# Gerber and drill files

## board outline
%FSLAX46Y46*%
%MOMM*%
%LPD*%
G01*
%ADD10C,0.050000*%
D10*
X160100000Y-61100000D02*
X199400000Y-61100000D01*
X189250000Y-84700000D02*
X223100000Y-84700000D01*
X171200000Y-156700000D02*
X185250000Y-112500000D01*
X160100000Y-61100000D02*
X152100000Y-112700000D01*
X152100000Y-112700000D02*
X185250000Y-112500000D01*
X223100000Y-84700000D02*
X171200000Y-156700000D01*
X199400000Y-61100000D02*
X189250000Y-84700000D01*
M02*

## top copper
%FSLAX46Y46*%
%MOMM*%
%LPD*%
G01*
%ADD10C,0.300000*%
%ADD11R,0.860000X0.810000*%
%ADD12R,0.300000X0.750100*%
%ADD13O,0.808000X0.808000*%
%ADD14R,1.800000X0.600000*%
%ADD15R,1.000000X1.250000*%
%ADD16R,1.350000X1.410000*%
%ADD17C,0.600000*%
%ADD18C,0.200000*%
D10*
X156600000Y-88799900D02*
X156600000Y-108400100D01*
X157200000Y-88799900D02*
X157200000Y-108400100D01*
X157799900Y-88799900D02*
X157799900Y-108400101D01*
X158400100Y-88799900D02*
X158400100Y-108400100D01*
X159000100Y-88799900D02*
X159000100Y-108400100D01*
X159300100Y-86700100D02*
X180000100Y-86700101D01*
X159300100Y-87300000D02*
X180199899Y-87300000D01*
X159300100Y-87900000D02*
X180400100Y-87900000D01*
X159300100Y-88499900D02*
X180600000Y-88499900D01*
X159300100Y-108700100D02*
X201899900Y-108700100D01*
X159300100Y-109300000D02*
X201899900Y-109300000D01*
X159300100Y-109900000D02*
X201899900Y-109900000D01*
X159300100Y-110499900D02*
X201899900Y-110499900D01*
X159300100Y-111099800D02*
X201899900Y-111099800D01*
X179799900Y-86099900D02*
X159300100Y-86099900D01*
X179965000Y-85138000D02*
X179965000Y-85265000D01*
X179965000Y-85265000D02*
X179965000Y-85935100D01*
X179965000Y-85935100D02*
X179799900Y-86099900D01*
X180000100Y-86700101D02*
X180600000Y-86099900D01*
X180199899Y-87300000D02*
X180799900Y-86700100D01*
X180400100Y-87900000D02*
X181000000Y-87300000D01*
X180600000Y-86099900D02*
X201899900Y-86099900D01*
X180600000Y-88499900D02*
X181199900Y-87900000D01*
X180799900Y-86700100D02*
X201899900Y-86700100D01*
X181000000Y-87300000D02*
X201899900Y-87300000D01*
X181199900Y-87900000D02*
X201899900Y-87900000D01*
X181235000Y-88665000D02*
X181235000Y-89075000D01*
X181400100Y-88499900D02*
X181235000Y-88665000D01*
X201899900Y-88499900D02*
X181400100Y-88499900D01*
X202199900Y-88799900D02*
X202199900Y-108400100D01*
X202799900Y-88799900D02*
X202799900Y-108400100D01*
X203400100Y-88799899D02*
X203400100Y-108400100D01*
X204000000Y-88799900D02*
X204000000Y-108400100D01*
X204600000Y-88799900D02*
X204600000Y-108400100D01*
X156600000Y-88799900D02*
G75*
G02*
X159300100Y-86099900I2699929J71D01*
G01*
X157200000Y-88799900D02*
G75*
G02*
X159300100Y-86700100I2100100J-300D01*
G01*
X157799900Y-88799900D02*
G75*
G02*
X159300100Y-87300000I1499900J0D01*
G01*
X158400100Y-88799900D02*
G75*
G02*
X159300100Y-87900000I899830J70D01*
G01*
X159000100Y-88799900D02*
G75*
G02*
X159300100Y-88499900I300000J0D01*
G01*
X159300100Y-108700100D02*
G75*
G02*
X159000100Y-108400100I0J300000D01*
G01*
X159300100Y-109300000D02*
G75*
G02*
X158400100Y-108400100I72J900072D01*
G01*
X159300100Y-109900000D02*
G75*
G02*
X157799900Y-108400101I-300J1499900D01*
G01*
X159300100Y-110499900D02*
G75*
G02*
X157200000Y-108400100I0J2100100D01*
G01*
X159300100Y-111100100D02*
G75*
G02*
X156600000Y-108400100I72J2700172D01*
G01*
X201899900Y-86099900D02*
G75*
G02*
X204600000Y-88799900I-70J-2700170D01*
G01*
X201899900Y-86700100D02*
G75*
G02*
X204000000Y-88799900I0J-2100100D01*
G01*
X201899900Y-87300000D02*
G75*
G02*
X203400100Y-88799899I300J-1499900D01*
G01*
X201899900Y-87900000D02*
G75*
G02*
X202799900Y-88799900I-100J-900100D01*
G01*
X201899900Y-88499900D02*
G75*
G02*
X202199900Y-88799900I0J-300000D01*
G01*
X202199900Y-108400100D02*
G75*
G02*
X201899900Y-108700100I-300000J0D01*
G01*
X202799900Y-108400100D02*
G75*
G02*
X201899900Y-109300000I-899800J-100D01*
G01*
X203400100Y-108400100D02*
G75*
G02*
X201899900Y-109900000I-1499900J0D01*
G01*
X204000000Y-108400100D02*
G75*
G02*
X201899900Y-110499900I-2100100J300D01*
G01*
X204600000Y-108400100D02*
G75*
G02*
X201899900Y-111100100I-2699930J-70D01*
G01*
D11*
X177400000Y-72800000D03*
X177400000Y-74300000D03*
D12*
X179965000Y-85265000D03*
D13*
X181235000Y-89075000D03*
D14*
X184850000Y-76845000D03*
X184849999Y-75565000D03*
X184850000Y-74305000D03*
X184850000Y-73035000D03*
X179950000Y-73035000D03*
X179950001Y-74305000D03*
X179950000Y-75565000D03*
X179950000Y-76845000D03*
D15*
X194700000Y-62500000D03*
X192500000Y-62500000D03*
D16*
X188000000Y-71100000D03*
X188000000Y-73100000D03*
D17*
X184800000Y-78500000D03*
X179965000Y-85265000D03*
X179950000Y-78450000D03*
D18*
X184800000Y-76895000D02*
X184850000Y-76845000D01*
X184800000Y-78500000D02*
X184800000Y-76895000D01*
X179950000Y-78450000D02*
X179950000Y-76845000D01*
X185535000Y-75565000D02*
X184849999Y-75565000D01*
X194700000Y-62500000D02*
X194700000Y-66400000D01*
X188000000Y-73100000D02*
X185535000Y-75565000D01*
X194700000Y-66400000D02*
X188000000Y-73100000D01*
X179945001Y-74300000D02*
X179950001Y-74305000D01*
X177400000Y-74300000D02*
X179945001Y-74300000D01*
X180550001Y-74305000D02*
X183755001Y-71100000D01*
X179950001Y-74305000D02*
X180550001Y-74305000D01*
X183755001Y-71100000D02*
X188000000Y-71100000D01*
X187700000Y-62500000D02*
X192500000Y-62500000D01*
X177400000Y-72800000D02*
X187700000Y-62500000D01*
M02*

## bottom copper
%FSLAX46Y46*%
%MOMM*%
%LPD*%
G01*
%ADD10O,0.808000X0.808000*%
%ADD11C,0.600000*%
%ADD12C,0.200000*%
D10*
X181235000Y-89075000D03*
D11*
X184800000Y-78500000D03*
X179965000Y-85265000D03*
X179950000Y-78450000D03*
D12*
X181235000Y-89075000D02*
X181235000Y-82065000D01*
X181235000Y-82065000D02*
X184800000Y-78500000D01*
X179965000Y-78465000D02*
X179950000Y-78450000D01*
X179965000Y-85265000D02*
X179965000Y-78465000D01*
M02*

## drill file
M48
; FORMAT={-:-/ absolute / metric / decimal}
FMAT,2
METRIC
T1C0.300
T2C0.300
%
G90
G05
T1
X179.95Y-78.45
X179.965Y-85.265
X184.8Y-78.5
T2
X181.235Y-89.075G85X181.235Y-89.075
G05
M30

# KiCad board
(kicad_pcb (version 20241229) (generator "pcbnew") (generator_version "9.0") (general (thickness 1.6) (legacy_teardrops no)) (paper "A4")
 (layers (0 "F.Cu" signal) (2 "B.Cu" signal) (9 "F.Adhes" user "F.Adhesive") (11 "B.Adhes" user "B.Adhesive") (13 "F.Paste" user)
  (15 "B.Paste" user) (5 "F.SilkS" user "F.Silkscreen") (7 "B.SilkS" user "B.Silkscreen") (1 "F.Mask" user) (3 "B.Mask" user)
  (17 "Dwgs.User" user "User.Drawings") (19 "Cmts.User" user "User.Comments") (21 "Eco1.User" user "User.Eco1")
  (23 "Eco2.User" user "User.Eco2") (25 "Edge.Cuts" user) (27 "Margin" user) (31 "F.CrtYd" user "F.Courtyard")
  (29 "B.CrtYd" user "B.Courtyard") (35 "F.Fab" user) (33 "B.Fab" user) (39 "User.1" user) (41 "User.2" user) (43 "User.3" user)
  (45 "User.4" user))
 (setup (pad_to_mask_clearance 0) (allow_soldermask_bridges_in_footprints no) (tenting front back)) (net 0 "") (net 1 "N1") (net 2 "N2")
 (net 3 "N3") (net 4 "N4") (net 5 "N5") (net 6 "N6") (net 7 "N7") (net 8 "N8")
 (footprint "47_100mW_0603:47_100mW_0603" (layer "F.Cu") (at 177.4 73.55 -90)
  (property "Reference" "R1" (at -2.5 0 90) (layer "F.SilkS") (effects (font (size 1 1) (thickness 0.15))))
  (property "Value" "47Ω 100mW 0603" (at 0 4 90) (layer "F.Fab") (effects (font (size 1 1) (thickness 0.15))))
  (pad "1" smd rect (at -0.75 0 270) (size 0.81 0.86) (layers "F.Cu" "F.Mask" "F.Paste") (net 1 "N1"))
  (pad "2" smd rect (at 0.75 0 270) (size 0.81 0.86) (layers "F.Cu" "F.Mask" "F.Paste") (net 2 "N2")))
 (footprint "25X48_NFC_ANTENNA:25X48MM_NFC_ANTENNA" (layer "F.Cu") (at 180.6 98.6)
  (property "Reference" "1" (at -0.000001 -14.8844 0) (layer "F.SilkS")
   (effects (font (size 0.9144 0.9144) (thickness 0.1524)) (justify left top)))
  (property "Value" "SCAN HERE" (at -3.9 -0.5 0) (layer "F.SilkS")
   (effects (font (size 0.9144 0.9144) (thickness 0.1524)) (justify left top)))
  (fp_line (start -24 -9.8001) (end -24 9.8001) (stroke (width 0.3) (type default)) (layer "F.Cu"))
  (fp_line (start -23.4 -9.8001) (end -23.4 9.8001) (stroke (width 0.3) (type default)) (layer "F.Cu"))
  (fp_line (start -22.8001 -9.8001) (end -22.8001 9.800101) (stroke (width 0.3) (type default)) (layer "F.Cu"))
  (fp_line (start -22.1999 -9.8001) (end -22.1999 9.8001) (stroke (width 0.3) (type default)) (layer "F.Cu"))
  (fp_line (start -21.5999 -9.8001) (end -21.5999 9.8001) (stroke (width 0.3) (type default)) (layer "F.Cu"))
  (fp_line (start -21.2999 -11.8999) (end -0.5999 -11.899899) (stroke (width 0.3) (type default)) (layer "F.Cu"))
  (fp_line (start -21.2999 -11.3) (end -0.400101 -11.3) (stroke (width 0.3) (type default)) (layer "F.Cu"))
  (fp_line (start -21.2999 -10.7) (end -0.1999 -10.7) (stroke (width 0.3) (type default)) (layer "F.Cu"))
  (fp_line (start -21.2999 -10.1001) (end 0 -10.1001) (stroke (width 0.3) (type default)) (layer "F.Cu"))
  (fp_line (start -21.2999 10.1001) (end 21.2999 10.1001) (stroke (width 0.3) (type default)) (layer "F.Cu"))
  (fp_line (start -21.2999 10.7) (end 21.2999 10.7) (stroke (width 0.3) (type default)) (layer "F.Cu"))
  (fp_line (start -21.2999 11.3) (end 21.2999 11.3) (stroke (width 0.3) (type default)) (layer "F.Cu"))
  (fp_line (start -21.2999 11.8999) (end 21.2999 11.8999) (stroke (width 0.3) (type default)) (layer "F.Cu"))
  (fp_line (start -21.2999 12.4998) (end 21.2999 12.4998) (stroke (width 0.3) (type default)) (layer "F.Cu"))
  (fp_line (start -0.8001 -12.5001) (end -21.2999 -12.5001) (stroke (width 0.3) (type default)) (layer "F.Cu"))
  (fp_line (start -0.635 -13.462) (end -0.635 -13.335) (stroke (width 0.3) (type default)) (layer "F.Cu"))
  (fp_line (start -0.635 -13.335) (end -0.635 -12.6649) (stroke (width 0.3) (type default)) (layer "F.Cu"))
  (fp_line (start -0.635 -12.6649) (end -0.8001 -12.5001) (stroke (width 0.3) (type default)) (layer "F.Cu"))
  (fp_line (start -0.5999 -11.899899) (end 0 -12.5001) (stroke (width 0.3) (type default)) (layer "F.Cu"))
  (fp_line (start -0.400101 -11.3) (end 0.1999 -11.8999) (stroke (width 0.3) (type default)) (layer "F.Cu"))
  (fp_line (start -0.1999 -10.7) (end 0.4 -11.3) (stroke (width 0.3) (type default)) (layer "F.Cu"))
  (fp_line (start 0 -12.5001) (end 21.2999 -12.5001) (stroke (width 0.3) (type default)) (layer "F.Cu"))
  (fp_line (start 0 -10.1001) (end 0.5999 -10.7) (stroke (width 0.3) (type default)) (layer "F.Cu"))
  (fp_line (start 0.1999 -11.8999) (end 21.2999 -11.8999) (stroke (width 0.3) (type default)) (layer "F.Cu"))
  (fp_line (start 0.4 -11.3) (end 21.2999 -11.3) (stroke (width 0.3) (type default)) (layer "F.Cu"))
  (fp_line (start 0.5999 -10.7) (end 21.2999 -10.7) (stroke (width 0.3) (type default)) (layer "F.Cu"))
  (fp_line (start 0.635 -9.935) (end 0.635 -9.525) (stroke (width 0.3) (type default)) (layer "F.Cu"))
  (fp_line (start 0.8001 -10.1001) (end 0.635 -9.935) (stroke (width 0.3) (type default)) (layer "F.Cu"))
  (fp_line (start 21.2999 -10.1001) (end 0.8001 -10.1001) (stroke (width 0.3) (type default)) (layer "F.Cu"))
  (fp_line (start 21.5999 -9.8001) (end 21.5999 9.8001) (stroke (width 0.3) (type default)) (layer "F.Cu"))
  (fp_line (start 22.1999 -9.8001) (end 22.1999 9.8001) (stroke (width 0.3) (type default)) (layer "F.Cu"))
  (fp_line (start 22.8001 -9.800101) (end 22.8001 9.8001) (stroke (width 0.3) (type default)) (layer "F.Cu"))
  (fp_line (start 23.4 -9.8001) (end 23.4 9.8001) (stroke (width 0.3) (type default)) (layer "F.Cu"))
  (fp_line (start 24 -9.8001) (end 24 9.8001) (stroke (width 0.3) (type default)) (layer "F.Cu"))
  (fp_arc (start -24 -9.8001) (mid -23.209159 -11.709359) (end -21.2999 -12.5001) (stroke (width 0.3) (type default)) (layer "F.Cu"))
  (fp_arc (start -23.4 -9.8001) (mid -22.784789 -11.284901) (end -21.2999 -11.8999) (stroke (width 0.3) (type default)) (layer "F.Cu"))
  (fp_arc (start -22.8001 -9.8001) (mid -22.360683 -10.860796) (end -21.2999 -11.3) (stroke (width 0.3) (type default)) (layer "F.Cu"))
  (fp_arc (start -22.1999 -9.8001) (mid -21.936296 -10.436496) (end -21.2999 -10.7) (stroke (width 0.3) (type default)) (layer "F.Cu"))
  (fp_arc (start -21.5999 -9.8001) (mid -21.512032 -10.012232) (end -21.2999 -10.1001) (stroke (width 0.3) (type default)) (layer "F.Cu"))
  (fp_arc (start -21.2999 10.1001) (mid -21.512032 10.012232) (end -21.5999 9.8001) (stroke (width 0.3) (type default)) (layer "F.Cu"))
  (fp_arc (start -21.2999 10.7) (mid -21.936225 10.436425) (end -22.1999 9.8001) (stroke (width 0.3) (type default)) (layer "F.Cu"))
  (fp_arc (start -21.2999 11.3) (mid -22.360683 10.860796) (end -22.8001 9.800101) (stroke (width 0.3) (type default)) (layer "F.Cu"))
  (fp_arc (start -21.2999 11.8999) (mid -22.784789 11.284901) (end -23.4 9.8001) (stroke (width 0.3) (type default)) (layer "F.Cu"))
  (fp_arc (start -21.2999 12.5001) (mid -23.209088 11.709288) (end -24 9.8001) (stroke (width 0.3) (type default)) (layer "F.Cu"))
  (fp_arc (start 21.2999 -12.5001) (mid 23.209088 -11.709288) (end 24 -9.8001) (stroke (width 0.3) (type default)) (layer "F.Cu"))
  (fp_arc (start 21.2999 -11.8999) (mid 22.784789 -11.284901) (end 23.4 -9.8001) (stroke (width 0.3) (type default)) (layer "F.Cu"))
  (fp_arc (start 21.2999 -11.3) (mid 22.360683 -10.860796) (end 22.8001 -9.800101) (stroke (width 0.3) (type default)) (layer "F.Cu"))
  (fp_arc (start 21.2999 -10.7) (mid 21.936225 -10.436425) (end 22.1999 -9.8001) (stroke (width 0.3) (type default)) (layer "F.Cu"))
  (fp_arc (start 21.2999 -10.1001) (mid 21.512032 -10.012232) (end 21.5999 -9.8001) (stroke (width 0.3) (type default)) (layer "F.Cu"))
  (fp_arc (start 21.5999 9.8001) (mid 21.512032 10.012232) (end 21.2999 10.1001) (stroke (width 0.3) (type default)) (layer "F.Cu"))
  (fp_arc (start 22.1999 9.8001) (mid 21.936296 10.436496) (end 21.2999 10.7) (stroke (width 0.3) (type default)) (layer "F.Cu"))
  (fp_arc (start 22.8001 9.8001) (mid 22.360683 10.860796) (end 21.2999 11.3) (stroke (width 0.3) (type default)) (layer "F.Cu"))
  (fp_arc (start 23.4 9.8001) (mid 22.784789 11.284901) (end 21.2999 11.8999) (stroke (width 0.3) (type default)) (layer "F.Cu"))
  (fp_arc (start 24 9.8001) (mid 23.209159 11.709359) (end 21.2999 12.5001) (stroke (width 0.3) (type default)) (layer "F.Cu"))
  (pad "P$1" smd rect (at -0.635 -13.335 90) (size 0.7501 0.3) (layers "F.Cu" "F.Mask" "F.Paste") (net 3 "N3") (solder_mask_margin 0.0508)
   (solder_paste_margin 0) (thermal_bridge_angle 0))
  (pad "P$2" thru_hole oval (at 0.635 -9.525) (size 0.808 0.808) (drill oval 0.3005 0.3002) (layers "*.Cu" "*.Mask")
   (remove_unused_layers no) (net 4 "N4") (solder_mask_margin 0.0508) (solder_paste_margin 0) (thermal_bridge_angle 0)))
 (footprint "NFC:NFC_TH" (layer "F.Cu") (at 182.4 74.935 90)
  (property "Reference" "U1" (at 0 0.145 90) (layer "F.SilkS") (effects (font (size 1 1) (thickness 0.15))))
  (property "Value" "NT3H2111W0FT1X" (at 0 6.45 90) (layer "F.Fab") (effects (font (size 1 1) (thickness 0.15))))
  (pad "1" smd rect (at -1.91 2.45 90) (size 0.6 1.8) (layers "F.Cu" "F.Mask" "F.Paste") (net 4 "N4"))
  (pad "2" smd rect (at -0.63 2.449999 90) (size 0.6 1.8) (layers "F.Cu" "F.Mask" "F.Paste") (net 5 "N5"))
  (pad "3" smd rect (at 0.63 2.45 90) (size 0.6 1.8) (layers "F.Cu" "F.Mask" "F.Paste") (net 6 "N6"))
  (pad "4" smd rect (at 1.9 2.45 90) (size 0.6 1.8) (layers "F.Cu" "F.Mask" "F.Paste") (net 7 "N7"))
  (pad "5" smd rect (at 1.9 -2.45 270) (size 0.6 1.8) (layers "F.Cu" "F.Mask" "F.Paste") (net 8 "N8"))
  (pad "6" smd rect (at 0.63 -2.449999 270) (size 0.6 1.8) (layers "F.Cu" "F.Mask" "F.Paste") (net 2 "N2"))
  (pad "7" smd rect (at -0.63 -2.45 270) (size 0.6 1.8) (layers "F.Cu" "F.Mask" "F.Paste") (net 2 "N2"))
  (pad "8" smd rect (at -1.91 -2.45 270) (size 0.6 1.8) (layers "F.Cu" "F.Mask" "F.Paste") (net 3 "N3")))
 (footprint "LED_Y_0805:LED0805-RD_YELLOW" (layer "F.Cu") (at 193.6 62.5 180)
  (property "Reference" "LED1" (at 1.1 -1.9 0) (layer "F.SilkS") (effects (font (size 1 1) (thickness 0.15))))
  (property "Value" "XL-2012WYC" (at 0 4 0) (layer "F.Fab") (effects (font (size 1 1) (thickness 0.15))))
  (pad "1" smd rect (at -1.1 0) (size 1 1.25) (layers "F.Cu" "F.Mask" "F.Paste") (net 5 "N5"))
  (pad "2" smd rect (at 1.1 0) (size 1 1.25) (layers "F.Cu" "F.Mask" "F.Paste") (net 1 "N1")))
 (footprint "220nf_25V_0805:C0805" (layer "F.Cu") (at 188 72.1 -90)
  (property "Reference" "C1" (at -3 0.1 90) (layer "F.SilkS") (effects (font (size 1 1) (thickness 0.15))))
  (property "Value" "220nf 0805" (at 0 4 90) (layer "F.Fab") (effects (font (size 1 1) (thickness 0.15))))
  (pad "1" smd rect (at -1 0 270) (size 1.41 1.35) (layers "F.Cu" "F.Mask" "F.Paste") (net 2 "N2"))
  (pad "2" smd rect (at 1 0 270) (size 1.41 1.35) (layers "F.Cu" "F.Mask" "F.Paste") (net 5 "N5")))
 (gr_line (start 160.1 61.1) (end 199.4 61.1) (stroke (width 0.05) (type default)) (layer "Edge.Cuts"))
 (gr_line (start 189.25 84.7) (end 223.1 84.7) (stroke (width 0.05) (type default)) (layer "Edge.Cuts"))
 (gr_line (start 171.2 156.7) (end 185.25 112.5) (stroke (width 0.05) (type default)) (layer "Edge.Cuts"))
 (gr_line (start 160.1 61.1) (end 152.1 112.7) (stroke (width 0.05) (type default)) (layer "Edge.Cuts"))
 (gr_line (start 152.1 112.7) (end 185.25 112.5) (stroke (width 0.05) (type default)) (layer "Edge.Cuts"))
 (gr_line (start 223.1 84.7) (end 171.2 156.7) (stroke (width 0.05) (type default)) (layer "Edge.Cuts"))
 (gr_line (start 199.4 61.1) (end 189.25 84.7) (stroke (width 0.05) (type default)) (layer "Edge.Cuts"))
 (segment (start 184.8 76.895) (end 184.85 76.845) (width 0.2) (layer "F.Cu") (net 4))
 (segment (start 184.8 78.5) (end 184.8 76.895) (width 0.2) (layer "F.Cu") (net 4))
 (via (at 184.8 78.5) (size 0.6) (drill 0.3) (layers "F.Cu" "B.Cu") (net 4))
 (segment (start 181.235 89.075) (end 181.235 82.065) (width 0.2) (layer "B.Cu") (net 4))
 (segment (start 181.235 82.065) (end 184.8 78.5) (width 0.2) (layer "B.Cu") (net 4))
 (segment (start 179.95 78.45) (end 179.95 76.845) (width 0.2) (layer "F.Cu") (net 3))
 (via (at 179.965 85.265) (size 0.6) (drill 0.3) (layers "F.Cu" "B.Cu") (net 3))
 (via (at 179.95 78.45) (size 0.6) (drill 0.3) (layers "F.Cu" "B.Cu") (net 3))
 (segment (start 179.965 78.465) (end 179.95 78.45) (width 0.2) (layer "B.Cu") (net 3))
 (segment (start 179.965 85.265) (end 179.965 78.465) (width 0.2) (layer "B.Cu") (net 3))
 (segment (start 185.535 75.565) (end 184.849999 75.565) (width 0.2) (layer "F.Cu") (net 5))
 (segment (start 194.7 62.5) (end 194.7 66.4) (width 0.2) (layer "F.Cu") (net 5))
 (segment (start 188 73.1) (end 185.535 75.565) (width 0.2) (layer "F.Cu") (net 5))
 (segment (start 194.7 66.4) (end 188 73.1) (width 0.2) (layer "F.Cu") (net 5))
 (segment (start 179.945001 74.3) (end 179.950001 74.305) (width 0.2) (layer "F.Cu") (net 2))
 (segment (start 177.4 74.3) (end 179.945001 74.3) (width 0.2) (layer "F.Cu") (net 2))
 (segment (start 180.550001 74.305) (end 183.755001 71.1) (width 0.2) (layer "F.Cu") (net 2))
 (segment (start 179.950001 74.305) (end 180.550001 74.305) (width 0.2) (layer "F.Cu") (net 2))
 (segment (start 183.755001 71.1) (end 188 71.1) (width 0.2) (layer "F.Cu") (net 2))
 (segment (start 187.7 62.5) (end 192.5 62.5) (width 0.2) (layer "F.Cu") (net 1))
 (segment (start 177.4 72.8) (end 187.7 62.5) (width 0.2) (layer "F.Cu") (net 1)))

